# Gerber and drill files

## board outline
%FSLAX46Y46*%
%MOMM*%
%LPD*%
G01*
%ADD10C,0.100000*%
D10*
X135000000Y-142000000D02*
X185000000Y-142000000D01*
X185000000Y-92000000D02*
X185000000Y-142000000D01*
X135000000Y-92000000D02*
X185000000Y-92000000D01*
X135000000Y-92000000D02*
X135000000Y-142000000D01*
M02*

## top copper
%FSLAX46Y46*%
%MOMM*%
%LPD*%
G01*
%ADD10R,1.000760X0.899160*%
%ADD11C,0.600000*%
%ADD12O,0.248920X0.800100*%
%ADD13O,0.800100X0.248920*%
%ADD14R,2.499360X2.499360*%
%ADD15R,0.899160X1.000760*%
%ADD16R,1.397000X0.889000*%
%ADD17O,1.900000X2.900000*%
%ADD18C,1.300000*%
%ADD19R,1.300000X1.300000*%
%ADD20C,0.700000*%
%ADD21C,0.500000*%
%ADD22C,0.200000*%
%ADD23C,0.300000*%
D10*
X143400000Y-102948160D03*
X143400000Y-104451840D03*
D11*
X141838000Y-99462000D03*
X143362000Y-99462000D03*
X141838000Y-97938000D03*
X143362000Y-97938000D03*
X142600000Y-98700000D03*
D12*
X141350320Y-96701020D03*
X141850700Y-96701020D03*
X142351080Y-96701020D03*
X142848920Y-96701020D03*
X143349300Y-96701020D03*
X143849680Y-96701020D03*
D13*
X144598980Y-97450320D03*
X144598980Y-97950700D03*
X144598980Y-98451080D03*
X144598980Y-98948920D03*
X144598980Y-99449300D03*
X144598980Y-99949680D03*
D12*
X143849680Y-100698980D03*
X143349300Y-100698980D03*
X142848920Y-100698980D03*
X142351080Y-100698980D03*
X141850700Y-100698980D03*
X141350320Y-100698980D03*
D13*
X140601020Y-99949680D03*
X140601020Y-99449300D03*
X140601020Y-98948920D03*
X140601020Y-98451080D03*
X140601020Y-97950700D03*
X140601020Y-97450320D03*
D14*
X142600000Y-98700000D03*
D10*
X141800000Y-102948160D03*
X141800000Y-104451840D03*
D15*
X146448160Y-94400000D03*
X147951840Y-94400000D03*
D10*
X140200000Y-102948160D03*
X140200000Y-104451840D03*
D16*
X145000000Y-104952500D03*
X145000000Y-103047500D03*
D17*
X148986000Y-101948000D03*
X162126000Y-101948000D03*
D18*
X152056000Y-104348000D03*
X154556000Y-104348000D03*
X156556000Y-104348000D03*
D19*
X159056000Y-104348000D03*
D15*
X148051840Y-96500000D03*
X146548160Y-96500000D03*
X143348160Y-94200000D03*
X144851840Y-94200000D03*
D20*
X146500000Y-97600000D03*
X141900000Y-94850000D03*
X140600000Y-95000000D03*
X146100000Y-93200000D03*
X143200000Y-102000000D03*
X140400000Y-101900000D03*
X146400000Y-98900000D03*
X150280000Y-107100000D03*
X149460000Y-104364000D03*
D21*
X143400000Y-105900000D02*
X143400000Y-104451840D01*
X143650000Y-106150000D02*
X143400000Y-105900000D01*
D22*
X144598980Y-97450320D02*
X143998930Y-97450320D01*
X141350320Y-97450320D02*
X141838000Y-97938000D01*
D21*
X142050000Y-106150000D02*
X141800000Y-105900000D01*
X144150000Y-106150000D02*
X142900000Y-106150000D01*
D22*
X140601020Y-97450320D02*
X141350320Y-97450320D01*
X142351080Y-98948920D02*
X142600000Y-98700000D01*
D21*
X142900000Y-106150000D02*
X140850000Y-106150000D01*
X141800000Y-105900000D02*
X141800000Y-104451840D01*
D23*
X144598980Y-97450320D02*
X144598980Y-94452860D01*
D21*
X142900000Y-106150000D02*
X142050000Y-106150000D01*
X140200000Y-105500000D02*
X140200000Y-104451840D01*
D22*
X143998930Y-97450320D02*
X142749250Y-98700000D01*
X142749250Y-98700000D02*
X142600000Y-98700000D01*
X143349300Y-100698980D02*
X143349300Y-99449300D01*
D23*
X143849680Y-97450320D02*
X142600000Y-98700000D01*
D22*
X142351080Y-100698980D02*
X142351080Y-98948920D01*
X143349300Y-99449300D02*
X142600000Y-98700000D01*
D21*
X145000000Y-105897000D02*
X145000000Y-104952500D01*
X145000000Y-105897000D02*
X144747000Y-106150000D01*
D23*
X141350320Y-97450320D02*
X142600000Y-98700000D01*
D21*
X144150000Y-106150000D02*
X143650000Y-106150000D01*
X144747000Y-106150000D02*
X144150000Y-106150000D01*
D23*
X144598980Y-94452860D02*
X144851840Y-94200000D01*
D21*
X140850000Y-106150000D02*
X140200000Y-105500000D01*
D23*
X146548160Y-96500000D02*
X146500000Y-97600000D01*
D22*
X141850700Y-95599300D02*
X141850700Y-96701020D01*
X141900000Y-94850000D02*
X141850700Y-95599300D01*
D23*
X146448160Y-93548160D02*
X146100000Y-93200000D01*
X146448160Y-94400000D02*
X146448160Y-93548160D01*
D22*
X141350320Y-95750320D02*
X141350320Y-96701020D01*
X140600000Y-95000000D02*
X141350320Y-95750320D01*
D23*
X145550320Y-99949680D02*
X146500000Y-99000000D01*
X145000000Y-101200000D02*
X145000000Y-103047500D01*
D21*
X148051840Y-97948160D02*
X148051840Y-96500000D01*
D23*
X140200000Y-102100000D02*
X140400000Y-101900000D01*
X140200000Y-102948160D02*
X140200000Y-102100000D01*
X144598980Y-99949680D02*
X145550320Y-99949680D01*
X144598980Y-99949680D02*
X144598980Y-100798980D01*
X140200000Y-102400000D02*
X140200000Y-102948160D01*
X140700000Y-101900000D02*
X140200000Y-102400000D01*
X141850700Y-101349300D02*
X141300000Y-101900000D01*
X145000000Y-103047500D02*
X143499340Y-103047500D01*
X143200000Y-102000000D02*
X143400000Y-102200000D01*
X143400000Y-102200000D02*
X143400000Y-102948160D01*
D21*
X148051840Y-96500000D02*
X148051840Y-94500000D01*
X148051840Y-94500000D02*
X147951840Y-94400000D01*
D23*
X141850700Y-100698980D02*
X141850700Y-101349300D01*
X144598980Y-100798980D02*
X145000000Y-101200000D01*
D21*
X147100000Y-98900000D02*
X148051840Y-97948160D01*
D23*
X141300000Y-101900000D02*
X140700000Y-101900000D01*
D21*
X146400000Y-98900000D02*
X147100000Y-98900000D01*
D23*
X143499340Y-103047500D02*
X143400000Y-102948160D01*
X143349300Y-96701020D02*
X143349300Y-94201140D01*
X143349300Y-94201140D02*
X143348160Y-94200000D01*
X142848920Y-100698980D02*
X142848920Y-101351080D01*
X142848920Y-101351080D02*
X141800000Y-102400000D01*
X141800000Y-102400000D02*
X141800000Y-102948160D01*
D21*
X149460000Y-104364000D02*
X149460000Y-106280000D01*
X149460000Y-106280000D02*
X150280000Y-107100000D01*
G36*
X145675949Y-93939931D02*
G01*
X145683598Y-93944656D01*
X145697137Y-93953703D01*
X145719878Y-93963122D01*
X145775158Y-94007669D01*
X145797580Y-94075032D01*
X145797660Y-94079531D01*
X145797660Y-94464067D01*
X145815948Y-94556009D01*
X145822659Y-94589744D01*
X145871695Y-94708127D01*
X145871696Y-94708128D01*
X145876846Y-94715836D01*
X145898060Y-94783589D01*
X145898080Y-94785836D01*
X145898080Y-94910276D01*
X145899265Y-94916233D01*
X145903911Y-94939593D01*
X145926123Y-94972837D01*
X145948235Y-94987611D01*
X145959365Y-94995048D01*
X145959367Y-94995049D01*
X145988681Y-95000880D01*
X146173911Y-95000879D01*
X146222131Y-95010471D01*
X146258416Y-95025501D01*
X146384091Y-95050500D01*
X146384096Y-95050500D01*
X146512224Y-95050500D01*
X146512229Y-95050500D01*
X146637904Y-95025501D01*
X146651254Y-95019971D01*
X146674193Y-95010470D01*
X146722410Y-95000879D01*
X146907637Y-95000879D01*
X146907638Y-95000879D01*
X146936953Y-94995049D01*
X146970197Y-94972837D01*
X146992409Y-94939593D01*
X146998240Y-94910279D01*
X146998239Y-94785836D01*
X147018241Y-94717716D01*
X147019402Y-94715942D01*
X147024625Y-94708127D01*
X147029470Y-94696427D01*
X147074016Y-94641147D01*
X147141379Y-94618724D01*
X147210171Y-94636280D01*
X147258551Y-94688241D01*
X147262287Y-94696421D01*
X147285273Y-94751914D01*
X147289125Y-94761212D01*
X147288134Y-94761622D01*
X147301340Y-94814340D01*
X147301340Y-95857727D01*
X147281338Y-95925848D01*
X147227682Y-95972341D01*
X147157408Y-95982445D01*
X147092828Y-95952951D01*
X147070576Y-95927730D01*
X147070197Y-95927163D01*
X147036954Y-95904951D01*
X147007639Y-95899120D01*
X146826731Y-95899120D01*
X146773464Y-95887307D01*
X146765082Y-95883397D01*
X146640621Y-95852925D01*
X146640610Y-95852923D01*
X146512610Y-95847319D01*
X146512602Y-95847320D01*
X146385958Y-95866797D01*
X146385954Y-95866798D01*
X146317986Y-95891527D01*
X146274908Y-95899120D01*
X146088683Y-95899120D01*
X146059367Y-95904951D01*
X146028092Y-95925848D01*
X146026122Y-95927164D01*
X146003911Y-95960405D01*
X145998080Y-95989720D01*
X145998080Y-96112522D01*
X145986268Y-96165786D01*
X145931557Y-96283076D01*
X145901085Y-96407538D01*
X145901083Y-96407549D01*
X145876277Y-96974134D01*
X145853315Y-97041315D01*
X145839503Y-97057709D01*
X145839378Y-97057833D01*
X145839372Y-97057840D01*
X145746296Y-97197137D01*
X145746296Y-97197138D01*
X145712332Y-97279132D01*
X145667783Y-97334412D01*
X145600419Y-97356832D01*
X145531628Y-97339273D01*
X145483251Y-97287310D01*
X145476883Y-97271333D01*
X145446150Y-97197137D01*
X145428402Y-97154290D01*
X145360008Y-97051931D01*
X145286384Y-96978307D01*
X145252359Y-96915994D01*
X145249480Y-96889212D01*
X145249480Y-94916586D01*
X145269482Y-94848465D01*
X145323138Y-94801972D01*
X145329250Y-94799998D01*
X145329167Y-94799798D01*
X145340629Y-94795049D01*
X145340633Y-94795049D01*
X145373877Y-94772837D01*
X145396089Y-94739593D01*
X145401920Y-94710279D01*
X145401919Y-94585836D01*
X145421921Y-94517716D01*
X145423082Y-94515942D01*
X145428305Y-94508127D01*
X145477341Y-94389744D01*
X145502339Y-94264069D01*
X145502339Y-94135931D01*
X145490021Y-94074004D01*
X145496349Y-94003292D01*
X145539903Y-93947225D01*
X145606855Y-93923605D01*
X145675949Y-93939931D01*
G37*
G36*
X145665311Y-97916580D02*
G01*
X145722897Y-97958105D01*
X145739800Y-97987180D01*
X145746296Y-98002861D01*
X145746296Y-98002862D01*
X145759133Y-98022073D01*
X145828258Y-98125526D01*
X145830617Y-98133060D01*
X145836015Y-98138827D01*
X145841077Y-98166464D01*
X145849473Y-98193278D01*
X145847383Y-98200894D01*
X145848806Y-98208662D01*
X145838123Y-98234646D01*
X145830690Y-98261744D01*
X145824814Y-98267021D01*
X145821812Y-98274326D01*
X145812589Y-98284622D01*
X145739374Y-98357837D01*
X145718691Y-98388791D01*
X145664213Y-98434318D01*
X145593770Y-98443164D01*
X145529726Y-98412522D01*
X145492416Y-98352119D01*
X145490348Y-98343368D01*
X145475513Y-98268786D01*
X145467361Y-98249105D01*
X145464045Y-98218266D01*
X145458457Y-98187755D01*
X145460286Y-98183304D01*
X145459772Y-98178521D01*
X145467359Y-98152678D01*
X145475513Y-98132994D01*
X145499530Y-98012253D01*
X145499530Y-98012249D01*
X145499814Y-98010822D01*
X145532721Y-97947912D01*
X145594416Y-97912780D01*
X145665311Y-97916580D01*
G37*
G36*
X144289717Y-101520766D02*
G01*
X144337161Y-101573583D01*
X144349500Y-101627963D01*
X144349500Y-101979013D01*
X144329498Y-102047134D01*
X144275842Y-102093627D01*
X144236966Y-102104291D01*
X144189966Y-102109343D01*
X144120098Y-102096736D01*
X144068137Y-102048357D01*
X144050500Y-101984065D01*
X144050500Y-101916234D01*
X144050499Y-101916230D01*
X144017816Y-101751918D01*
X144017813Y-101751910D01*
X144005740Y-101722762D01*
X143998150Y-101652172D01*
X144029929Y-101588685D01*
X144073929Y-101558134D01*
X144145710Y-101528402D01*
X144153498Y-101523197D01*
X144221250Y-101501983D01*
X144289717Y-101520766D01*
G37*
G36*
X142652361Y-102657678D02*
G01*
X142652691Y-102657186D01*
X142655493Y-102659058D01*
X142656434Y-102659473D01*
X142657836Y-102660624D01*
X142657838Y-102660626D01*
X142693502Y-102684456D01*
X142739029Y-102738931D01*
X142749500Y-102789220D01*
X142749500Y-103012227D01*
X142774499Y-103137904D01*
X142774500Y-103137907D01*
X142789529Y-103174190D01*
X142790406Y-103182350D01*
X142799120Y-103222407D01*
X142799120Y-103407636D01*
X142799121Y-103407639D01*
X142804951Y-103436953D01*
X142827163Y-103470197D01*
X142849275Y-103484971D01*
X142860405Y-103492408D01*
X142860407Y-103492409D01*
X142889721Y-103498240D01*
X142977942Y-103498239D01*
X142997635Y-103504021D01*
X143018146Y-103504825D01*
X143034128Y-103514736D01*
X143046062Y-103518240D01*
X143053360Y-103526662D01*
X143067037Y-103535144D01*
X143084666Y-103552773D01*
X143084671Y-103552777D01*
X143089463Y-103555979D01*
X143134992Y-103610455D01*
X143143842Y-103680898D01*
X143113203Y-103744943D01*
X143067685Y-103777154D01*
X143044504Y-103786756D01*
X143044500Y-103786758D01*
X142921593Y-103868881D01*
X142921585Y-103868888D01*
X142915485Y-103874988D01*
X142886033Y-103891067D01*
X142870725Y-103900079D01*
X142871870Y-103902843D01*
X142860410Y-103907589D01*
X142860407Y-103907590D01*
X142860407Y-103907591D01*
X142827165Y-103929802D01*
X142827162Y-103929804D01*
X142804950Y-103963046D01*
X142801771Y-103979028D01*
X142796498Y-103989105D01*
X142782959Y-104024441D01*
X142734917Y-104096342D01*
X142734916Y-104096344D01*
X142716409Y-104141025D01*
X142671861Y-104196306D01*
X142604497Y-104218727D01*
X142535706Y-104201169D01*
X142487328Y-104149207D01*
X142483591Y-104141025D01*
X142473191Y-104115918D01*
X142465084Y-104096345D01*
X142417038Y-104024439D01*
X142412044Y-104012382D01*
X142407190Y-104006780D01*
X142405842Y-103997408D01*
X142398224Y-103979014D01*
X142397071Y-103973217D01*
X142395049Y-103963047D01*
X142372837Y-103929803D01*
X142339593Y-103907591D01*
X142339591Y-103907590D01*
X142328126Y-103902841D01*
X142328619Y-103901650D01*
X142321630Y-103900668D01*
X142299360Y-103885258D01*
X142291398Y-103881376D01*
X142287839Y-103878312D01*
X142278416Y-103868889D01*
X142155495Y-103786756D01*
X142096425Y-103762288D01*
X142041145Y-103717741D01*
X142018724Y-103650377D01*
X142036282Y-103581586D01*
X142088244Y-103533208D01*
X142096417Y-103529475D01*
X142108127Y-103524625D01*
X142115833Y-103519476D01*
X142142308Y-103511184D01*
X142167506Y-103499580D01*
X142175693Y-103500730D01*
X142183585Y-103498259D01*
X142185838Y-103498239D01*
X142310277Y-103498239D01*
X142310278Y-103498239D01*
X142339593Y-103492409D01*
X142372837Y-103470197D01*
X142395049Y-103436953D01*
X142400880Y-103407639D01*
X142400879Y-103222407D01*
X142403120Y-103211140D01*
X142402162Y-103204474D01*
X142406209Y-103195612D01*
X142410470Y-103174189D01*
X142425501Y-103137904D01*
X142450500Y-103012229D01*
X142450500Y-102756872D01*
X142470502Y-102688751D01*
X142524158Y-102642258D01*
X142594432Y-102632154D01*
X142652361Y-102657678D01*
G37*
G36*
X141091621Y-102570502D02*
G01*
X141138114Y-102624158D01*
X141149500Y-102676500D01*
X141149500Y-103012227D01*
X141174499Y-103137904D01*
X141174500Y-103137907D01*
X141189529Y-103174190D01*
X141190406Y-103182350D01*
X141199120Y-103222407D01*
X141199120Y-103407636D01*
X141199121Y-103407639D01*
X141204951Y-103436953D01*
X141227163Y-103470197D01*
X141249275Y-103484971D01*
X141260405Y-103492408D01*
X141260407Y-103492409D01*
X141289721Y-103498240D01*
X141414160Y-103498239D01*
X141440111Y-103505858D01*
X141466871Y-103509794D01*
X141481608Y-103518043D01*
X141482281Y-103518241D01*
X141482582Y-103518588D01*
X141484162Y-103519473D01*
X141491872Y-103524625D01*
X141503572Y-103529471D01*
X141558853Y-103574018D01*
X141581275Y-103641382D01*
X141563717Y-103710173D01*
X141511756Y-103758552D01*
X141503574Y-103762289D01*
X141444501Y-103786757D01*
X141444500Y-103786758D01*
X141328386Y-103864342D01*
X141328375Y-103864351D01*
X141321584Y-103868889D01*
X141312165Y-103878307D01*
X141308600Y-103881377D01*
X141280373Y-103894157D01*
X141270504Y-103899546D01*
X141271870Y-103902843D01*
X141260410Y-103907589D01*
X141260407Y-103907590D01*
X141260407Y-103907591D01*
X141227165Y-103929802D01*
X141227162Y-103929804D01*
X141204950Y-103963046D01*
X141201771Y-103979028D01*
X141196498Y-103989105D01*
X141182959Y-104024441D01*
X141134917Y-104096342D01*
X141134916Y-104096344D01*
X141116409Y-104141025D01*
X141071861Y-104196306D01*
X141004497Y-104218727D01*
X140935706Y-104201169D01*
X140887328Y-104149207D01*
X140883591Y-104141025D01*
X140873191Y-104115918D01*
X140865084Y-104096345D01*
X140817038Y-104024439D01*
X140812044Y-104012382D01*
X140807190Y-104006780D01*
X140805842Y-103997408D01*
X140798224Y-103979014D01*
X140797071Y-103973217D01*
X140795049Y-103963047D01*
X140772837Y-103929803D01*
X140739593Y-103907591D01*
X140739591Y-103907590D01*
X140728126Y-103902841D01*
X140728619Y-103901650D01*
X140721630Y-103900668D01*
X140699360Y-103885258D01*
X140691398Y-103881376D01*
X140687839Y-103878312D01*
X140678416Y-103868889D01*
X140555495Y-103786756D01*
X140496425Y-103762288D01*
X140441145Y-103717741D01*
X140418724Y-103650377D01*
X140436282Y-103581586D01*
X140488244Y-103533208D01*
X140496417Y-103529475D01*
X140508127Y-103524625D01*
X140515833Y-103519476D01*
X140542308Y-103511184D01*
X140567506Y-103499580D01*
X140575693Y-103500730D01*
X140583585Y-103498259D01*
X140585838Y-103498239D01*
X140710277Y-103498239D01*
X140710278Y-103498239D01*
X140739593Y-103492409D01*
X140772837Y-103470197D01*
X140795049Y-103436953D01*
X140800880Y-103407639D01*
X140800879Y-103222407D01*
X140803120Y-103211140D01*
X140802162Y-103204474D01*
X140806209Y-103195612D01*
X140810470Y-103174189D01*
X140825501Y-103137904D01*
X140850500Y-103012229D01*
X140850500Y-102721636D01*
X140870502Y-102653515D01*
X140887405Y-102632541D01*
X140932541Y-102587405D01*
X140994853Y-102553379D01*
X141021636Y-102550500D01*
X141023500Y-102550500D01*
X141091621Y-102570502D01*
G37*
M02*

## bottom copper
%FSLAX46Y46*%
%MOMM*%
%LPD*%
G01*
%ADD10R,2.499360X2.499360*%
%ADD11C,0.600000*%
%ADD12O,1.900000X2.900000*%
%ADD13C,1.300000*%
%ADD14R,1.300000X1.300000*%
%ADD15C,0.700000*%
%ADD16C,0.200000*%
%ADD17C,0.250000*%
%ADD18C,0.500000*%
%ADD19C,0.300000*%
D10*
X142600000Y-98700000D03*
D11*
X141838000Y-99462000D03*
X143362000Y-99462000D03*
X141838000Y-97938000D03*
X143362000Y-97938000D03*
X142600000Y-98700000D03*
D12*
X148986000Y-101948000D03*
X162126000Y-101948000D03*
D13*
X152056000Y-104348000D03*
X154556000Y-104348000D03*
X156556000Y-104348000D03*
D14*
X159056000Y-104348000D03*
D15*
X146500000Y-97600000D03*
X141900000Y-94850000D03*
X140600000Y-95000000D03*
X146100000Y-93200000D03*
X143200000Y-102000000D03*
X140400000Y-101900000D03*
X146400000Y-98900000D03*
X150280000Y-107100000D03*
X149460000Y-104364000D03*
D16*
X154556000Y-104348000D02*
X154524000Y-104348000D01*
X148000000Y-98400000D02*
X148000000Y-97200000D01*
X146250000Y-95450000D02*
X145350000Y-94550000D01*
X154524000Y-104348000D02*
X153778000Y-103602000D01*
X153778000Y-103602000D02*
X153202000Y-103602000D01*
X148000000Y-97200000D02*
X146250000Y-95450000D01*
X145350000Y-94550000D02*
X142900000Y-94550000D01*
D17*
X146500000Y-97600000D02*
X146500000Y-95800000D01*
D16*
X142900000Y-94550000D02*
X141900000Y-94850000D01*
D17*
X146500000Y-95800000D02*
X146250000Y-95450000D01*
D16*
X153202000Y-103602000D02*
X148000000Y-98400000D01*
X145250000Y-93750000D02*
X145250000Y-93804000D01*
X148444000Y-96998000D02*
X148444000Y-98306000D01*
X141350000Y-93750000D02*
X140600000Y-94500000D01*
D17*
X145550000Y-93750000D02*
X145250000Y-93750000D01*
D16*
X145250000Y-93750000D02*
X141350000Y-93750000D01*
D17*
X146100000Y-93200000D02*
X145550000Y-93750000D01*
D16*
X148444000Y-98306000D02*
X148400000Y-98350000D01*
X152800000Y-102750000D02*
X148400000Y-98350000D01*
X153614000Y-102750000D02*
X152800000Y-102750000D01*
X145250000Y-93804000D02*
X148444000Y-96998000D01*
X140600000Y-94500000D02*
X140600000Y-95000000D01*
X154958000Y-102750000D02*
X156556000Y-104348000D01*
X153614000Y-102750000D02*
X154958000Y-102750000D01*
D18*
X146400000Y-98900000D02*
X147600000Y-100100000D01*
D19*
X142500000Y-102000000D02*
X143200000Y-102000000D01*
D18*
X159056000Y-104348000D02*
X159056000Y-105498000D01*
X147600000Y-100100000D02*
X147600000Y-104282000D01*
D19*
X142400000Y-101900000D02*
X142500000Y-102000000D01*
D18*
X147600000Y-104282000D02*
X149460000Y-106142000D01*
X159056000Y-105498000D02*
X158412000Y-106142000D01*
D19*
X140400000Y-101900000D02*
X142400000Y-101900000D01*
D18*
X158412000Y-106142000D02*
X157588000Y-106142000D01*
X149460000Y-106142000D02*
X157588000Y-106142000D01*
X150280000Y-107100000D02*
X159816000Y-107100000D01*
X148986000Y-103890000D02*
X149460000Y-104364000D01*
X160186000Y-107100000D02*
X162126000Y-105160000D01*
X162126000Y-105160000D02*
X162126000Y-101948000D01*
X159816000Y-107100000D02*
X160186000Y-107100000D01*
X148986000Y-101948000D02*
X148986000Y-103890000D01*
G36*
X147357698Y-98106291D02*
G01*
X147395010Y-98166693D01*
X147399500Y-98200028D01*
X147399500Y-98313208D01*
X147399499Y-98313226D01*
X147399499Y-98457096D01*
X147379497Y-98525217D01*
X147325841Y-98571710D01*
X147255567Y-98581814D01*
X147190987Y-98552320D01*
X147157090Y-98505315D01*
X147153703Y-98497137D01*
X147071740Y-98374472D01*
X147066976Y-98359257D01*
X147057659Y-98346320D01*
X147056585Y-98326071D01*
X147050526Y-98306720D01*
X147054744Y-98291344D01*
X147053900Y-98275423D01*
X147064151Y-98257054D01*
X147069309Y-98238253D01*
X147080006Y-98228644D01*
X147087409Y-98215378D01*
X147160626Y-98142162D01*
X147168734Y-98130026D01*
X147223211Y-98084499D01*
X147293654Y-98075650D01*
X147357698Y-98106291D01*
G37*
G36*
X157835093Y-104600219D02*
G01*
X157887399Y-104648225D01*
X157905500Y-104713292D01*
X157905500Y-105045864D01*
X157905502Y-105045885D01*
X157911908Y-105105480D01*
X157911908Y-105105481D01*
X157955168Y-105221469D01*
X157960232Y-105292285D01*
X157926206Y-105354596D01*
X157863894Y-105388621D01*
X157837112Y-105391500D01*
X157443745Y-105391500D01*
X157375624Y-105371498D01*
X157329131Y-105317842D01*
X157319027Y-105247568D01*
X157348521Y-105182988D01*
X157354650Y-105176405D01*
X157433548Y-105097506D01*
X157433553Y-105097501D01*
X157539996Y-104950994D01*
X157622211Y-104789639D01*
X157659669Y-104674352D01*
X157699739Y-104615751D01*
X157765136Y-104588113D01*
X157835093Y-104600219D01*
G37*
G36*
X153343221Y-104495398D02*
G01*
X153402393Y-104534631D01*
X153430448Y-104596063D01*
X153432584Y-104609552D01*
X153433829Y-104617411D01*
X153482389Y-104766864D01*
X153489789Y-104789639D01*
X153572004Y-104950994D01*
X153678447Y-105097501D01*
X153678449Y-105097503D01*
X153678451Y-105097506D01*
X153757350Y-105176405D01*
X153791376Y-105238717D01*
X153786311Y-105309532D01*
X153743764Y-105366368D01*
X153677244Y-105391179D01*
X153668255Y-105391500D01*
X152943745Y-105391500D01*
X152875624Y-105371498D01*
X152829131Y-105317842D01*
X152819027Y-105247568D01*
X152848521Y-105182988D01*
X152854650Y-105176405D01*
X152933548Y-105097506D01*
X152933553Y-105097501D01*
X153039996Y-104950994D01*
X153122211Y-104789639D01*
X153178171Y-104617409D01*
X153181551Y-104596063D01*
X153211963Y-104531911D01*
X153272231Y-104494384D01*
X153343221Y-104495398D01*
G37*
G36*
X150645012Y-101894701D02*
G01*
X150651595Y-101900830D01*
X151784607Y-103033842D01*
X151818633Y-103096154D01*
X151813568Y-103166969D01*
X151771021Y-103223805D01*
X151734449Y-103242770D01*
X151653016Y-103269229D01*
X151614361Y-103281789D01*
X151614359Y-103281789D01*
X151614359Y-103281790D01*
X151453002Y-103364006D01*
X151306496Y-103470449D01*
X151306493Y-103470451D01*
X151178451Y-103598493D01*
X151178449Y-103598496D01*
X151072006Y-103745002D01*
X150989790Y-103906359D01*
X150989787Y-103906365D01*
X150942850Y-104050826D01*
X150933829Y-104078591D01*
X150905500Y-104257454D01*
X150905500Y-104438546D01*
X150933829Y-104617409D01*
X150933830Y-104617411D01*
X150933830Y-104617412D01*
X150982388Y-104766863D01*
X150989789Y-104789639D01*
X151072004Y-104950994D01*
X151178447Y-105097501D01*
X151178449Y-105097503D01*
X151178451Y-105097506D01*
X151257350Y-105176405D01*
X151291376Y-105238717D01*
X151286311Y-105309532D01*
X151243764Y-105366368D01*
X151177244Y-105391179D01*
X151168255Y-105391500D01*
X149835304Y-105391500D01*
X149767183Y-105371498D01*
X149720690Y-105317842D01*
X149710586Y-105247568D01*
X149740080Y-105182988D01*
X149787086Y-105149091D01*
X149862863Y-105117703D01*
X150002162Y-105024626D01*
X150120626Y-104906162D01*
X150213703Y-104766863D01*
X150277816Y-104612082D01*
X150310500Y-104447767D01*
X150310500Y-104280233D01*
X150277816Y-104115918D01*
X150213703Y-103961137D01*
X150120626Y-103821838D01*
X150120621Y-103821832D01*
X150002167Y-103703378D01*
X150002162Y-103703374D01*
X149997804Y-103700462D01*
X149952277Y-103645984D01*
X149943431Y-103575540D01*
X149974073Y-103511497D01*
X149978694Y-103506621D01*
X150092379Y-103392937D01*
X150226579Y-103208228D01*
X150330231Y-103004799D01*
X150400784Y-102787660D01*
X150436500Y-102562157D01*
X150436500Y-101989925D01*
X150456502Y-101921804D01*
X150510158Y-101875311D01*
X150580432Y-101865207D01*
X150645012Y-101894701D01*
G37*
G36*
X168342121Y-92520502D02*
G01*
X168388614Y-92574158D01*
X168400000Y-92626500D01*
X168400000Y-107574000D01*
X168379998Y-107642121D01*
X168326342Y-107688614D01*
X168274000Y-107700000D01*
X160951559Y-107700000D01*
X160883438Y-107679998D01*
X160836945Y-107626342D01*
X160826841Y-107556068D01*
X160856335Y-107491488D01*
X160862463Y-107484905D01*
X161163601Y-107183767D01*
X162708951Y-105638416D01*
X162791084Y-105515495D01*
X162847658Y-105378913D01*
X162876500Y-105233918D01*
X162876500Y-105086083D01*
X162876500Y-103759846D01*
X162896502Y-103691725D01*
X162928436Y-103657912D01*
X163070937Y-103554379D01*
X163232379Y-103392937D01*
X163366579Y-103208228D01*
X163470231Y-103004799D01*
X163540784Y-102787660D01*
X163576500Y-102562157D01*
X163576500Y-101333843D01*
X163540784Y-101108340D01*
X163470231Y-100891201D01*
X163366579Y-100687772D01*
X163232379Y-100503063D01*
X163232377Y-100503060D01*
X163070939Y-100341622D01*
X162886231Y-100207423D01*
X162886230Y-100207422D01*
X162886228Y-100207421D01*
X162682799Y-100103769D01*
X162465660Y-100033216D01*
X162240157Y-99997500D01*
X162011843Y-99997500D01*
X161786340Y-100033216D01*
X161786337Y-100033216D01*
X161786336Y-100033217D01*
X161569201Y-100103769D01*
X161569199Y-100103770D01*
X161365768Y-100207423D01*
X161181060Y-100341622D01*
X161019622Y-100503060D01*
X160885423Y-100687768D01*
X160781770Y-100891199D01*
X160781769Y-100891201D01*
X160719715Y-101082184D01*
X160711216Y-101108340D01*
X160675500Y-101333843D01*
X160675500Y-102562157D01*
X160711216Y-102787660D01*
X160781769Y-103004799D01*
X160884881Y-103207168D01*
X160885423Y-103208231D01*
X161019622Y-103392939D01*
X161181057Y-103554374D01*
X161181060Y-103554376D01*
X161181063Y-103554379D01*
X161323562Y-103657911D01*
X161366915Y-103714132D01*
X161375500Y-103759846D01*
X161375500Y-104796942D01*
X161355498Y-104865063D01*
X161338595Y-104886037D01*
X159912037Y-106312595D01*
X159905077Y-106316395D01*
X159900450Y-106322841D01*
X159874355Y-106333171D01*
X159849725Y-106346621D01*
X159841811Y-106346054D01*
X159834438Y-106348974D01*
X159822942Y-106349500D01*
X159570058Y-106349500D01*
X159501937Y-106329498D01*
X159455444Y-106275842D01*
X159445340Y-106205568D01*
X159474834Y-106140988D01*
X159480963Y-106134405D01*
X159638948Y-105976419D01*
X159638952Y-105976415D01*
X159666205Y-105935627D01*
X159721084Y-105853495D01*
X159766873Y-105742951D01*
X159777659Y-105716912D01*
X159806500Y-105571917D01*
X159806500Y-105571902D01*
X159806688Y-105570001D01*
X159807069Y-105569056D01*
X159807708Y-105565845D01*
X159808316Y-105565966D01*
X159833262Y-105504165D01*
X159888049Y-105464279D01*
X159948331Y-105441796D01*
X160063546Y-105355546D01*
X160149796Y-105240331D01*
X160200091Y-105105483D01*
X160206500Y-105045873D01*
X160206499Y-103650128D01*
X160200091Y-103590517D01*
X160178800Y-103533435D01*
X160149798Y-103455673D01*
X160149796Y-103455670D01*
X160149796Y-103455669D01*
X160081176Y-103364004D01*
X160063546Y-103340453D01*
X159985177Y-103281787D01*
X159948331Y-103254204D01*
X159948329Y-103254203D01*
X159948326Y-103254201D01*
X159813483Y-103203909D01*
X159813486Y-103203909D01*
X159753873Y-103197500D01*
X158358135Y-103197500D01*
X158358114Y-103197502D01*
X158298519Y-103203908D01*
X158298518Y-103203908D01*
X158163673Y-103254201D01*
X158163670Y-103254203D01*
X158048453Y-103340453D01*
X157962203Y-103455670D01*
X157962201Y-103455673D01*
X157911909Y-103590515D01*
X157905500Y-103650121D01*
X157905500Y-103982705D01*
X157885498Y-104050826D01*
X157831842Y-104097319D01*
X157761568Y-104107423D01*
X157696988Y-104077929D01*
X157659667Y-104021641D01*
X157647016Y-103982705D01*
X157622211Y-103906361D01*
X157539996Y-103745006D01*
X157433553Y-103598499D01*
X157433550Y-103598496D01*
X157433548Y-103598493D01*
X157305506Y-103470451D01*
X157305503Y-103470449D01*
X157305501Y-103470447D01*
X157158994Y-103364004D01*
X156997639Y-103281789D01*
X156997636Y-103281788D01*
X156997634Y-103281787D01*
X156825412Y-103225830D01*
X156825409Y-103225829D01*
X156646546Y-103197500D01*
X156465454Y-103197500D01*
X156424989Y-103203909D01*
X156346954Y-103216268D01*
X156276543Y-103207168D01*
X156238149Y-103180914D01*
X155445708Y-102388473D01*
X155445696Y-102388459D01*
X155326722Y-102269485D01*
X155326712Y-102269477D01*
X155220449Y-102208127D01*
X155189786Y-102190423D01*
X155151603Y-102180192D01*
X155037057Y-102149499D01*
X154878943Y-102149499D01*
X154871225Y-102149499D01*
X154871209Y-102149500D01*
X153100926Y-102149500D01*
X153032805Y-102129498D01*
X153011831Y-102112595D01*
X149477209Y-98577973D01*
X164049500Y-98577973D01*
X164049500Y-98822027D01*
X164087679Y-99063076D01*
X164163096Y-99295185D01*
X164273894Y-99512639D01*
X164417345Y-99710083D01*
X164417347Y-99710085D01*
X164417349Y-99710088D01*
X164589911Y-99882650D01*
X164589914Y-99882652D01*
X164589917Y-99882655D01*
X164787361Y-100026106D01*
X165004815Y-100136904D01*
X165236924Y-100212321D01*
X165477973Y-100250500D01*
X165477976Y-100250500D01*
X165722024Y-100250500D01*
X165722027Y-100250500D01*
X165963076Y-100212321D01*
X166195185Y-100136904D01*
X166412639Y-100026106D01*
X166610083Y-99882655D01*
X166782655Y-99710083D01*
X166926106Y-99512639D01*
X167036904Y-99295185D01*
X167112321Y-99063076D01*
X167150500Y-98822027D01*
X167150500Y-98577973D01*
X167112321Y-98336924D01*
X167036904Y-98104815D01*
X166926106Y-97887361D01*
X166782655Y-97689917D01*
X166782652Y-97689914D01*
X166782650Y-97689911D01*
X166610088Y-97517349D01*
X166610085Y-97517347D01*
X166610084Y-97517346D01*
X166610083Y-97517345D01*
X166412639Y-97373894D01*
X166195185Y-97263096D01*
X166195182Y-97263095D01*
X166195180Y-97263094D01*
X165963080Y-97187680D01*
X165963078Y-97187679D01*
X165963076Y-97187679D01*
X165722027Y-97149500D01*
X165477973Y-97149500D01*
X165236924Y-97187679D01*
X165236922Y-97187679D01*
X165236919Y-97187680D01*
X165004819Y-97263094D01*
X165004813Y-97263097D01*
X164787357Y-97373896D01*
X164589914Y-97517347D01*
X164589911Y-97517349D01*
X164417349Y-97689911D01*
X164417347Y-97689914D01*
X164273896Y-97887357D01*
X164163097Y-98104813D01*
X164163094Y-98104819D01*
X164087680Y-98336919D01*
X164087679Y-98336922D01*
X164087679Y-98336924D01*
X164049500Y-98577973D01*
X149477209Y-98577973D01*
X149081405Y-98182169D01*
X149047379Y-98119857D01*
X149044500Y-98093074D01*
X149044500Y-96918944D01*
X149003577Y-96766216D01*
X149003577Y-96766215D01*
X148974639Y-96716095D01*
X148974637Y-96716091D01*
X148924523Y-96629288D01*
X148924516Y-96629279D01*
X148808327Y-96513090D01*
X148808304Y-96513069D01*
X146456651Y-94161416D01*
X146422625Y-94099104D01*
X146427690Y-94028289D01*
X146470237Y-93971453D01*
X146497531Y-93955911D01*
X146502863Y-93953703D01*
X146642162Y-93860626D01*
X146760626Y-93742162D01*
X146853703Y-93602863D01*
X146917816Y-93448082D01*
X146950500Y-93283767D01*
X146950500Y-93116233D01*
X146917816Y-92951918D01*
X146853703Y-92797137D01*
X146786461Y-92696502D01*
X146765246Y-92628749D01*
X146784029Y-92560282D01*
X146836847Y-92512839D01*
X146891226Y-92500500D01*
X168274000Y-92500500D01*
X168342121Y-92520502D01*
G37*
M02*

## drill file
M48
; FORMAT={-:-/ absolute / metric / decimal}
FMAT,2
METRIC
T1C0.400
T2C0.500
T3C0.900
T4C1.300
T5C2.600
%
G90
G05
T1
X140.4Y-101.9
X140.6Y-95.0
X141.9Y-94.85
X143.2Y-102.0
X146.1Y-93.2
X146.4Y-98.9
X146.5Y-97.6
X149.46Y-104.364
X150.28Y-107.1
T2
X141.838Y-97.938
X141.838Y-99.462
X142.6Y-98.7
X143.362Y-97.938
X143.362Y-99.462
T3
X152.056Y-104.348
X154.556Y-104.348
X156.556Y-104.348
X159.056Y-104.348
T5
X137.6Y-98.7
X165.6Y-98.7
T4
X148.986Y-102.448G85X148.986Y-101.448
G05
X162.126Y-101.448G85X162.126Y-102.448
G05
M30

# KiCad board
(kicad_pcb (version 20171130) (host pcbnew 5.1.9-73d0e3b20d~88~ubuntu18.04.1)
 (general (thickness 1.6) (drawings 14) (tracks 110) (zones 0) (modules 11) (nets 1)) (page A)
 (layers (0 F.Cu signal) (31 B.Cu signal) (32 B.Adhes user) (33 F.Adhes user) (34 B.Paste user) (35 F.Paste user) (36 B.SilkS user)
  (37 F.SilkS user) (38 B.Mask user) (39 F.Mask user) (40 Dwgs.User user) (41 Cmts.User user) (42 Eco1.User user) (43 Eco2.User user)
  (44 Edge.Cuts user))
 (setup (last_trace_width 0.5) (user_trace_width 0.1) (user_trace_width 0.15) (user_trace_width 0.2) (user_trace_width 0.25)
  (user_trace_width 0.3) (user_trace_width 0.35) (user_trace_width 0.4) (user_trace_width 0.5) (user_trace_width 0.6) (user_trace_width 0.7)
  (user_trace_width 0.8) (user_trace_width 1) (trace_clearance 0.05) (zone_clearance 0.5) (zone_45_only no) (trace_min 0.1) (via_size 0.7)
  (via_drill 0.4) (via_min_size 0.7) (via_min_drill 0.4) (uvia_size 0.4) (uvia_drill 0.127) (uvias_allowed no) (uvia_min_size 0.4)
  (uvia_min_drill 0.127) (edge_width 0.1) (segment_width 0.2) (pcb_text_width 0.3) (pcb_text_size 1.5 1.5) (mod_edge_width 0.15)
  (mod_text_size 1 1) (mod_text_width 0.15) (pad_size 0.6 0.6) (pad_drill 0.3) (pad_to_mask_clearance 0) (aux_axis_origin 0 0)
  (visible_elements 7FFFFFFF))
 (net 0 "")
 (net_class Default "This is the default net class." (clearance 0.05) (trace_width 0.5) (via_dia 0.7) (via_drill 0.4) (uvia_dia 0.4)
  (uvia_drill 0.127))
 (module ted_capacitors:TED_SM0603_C (layer F.Cu) (at 143.4 103.7 270)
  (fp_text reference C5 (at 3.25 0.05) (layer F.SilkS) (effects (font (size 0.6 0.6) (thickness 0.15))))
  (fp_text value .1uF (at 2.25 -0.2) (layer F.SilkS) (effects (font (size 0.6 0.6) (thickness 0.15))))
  (pad 1 smd rect (at -0.75184 0 270) (size 0.89916 1.00076) (layers F.Cu F.Paste F.Mask) (clearance 0.1))
  (pad 2 smd rect (at 0.75184 0 270) (size 0.89916 1.00076) (layers F.Cu F.Paste F.Mask) (clearance 0.1)))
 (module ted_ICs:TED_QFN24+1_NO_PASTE (layer F.Cu) (at 142.6 98.7)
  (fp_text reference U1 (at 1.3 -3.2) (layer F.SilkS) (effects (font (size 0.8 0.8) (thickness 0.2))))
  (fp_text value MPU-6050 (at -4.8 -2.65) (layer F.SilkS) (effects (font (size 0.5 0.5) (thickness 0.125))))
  (pad 25 smd rect (at 0 0 270) (size 2.49936 2.49936) (layers B.Cu B.Mask) (zone_connect 2))
  (pad 25 thru_hole circle (at -0.762 0.762 270) (size 0.6 0.6) (drill 0.5) (layers *.Cu) (zone_connect 2))
  (pad 25 thru_hole circle (at 0.762 0.762 270) (size 0.6 0.6) (drill 0.5) (layers *.Cu) (zone_connect 2))
  (pad 25 thru_hole circle (at -0.762 -0.762 270) (size 0.6 0.6) (drill 0.5) (layers *.Cu) (zone_connect 2))
  (pad 25 thru_hole circle (at 0.762 -0.762 270) (size 0.6 0.6) (drill 0.5) (layers *.Cu) (zone_connect 2))
  (pad 25 thru_hole circle (at 0 0 270) (size 0.6 0.6) (drill 0.5) (layers *.Cu) (zone_connect 2))
  (pad 24 smd oval (at -1.24968 -1.99898 270) (size 0.8001 0.24892) (layers F.Cu F.Paste F.Mask))
  (pad 23 smd oval (at -0.7493 -1.99898 270) (size 0.8001 0.24892) (layers F.Cu F.Paste F.Mask))
  (pad 22 smd oval (at -0.24892 -1.99898 270) (size 0.8001 0.24892) (layers F.Cu F.Paste F.Mask))
  (pad 21 smd oval (at 0.24892 -1.99898 270) (size 0.8001 0.24892) (layers F.Cu F.Paste F.Mask))
  (pad 20 smd oval (at 0.7493 -1.99898 270) (size 0.8001 0.24892) (layers F.Cu F.Paste F.Mask))
  (pad 19 smd oval (at 1.24968 -1.99898 270) (size 0.8001 0.24892) (layers F.Cu F.Paste F.Mask))
  (pad 18 smd oval (at 1.99898 -1.24968 180) (size 0.8001 0.24892) (layers F.Cu F.Paste F.Mask))
  (pad 17 smd oval (at 1.99898 -0.7493 180) (size 0.8001 0.24892) (layers F.Cu F.Paste F.Mask))
  (pad 16 smd oval (at 1.99898 -0.24892 180) (size 0.8001 0.24892) (layers F.Cu F.Paste F.Mask))
  (pad 15 smd oval (at 1.99898 0.24892 180) (size 0.8001 0.24892) (layers F.Cu F.Paste F.Mask))
  (pad 14 smd oval (at 1.99898 0.7493 180) (size 0.8001 0.24892) (layers F.Cu F.Paste F.Mask))
  (pad 13 smd oval (at 1.99898 1.24968 180) (size 0.8001 0.24892) (layers F.Cu F.Paste F.Mask))
  (pad 12 smd oval (at 1.24968 1.99898 90) (size 0.8001 0.24892) (layers F.Cu F.Paste F.Mask))
  (pad 11 smd oval (at 0.7493 1.99898 90) (size 0.8001 0.24892) (layers F.Cu F.Paste F.Mask))
  (pad 10 smd oval (at 0.24892 1.99898 90) (size 0.8001 0.24892) (layers F.Cu F.Paste F.Mask))
  (pad 9 smd oval (at -0.24892 1.99898 90) (size 0.8001 0.24892) (layers F.Cu F.Paste F.Mask))
  (pad 8 smd oval (at -0.7493 1.99898 90) (size 0.8001 0.24892) (layers F.Cu F.Paste F.Mask))
  (pad 7 smd oval (at -1.24968 1.99898 90) (size 0.8001 0.24892) (layers F.Cu F.Paste F.Mask))
  (pad 6 smd oval (at -1.99898 1.24968) (size 0.8001 0.24892) (layers F.Cu F.Paste F.Mask))
  (pad 5 smd oval (at -1.99898 0.7493) (size 0.8001 0.24892) (layers F.Cu F.Paste F.Mask))
  (pad 4 smd oval (at -1.99898 0.24892) (size 0.8001 0.24892) (layers F.Cu F.Paste F.Mask))
  (pad 3 smd oval (at -1.99898 -0.24892) (size 0.8001 0.24892) (layers F.Cu F.Paste F.Mask))
  (pad 2 smd oval (at -1.99898 -0.7493) (size 0.8001 0.24892) (layers F.Cu F.Paste F.Mask))
  (pad 1 smd oval (at -1.99898 -1.24968) (size 0.8001 0.24892) (layers F.Cu F.Paste F.Mask))
  (pad 25 smd rect (at 0 0 270) (size 2.49936 2.49936) (layers F.Cu F.Mask) (zone_connect 2)))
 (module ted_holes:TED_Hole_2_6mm (layer F.Cu) (at 165.6 98.7)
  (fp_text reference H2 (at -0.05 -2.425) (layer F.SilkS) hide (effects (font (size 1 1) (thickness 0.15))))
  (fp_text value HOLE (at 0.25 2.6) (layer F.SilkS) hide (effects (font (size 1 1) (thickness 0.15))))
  (pad "" np_thru_hole circle (at 0 0) (size 2.6 2.6) (drill 2.6) (layers *.Cu *.Mask F.SilkS)))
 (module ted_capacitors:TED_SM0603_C (layer F.Cu) (at 141.8 103.7 270)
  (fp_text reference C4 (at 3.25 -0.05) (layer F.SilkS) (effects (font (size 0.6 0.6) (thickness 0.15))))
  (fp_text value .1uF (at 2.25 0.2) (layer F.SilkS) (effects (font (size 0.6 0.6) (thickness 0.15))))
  (pad 1 smd rect (at -0.75184 0 270) (size 0.89916 1.00076) (layers F.Cu F.Paste F.Mask) (clearance 0.1))
  (pad 2 smd rect (at 0.75184 0 270) (size 0.89916 1.00076) (layers F.Cu F.Paste F.Mask) (clearance 0.1)))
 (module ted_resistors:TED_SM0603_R (layer F.Cu) (at 147.2 94.4 180)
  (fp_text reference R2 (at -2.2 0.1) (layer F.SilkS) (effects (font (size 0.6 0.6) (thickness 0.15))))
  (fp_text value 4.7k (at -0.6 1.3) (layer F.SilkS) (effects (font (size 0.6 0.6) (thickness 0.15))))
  (pad 2 smd rect (at 0.75184 0 180) (size 0.89916 1.00076) (layers F.Cu F.Paste F.Mask) (clearance 0.1))
  (pad 1 smd rect (at -0.75184 0 180) (size 0.89916 1.00076) (layers F.Cu F.Paste F.Mask) (clearance 0.1)))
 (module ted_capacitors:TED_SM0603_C (layer F.Cu) (at 140.2 103.7 270)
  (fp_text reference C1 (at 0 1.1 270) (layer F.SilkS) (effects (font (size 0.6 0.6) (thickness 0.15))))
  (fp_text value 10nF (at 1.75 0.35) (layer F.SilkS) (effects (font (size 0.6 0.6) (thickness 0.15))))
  (pad 1 smd rect (at -0.75184 0 270) (size 0.89916 1.00076) (layers F.Cu F.Paste F.Mask) (clearance 0.1))
  (pad 2 smd rect (at 0.75184 0 270) (size 0.89916 1.00076) (layers F.Cu F.Paste F.Mask) (clearance 0.1)))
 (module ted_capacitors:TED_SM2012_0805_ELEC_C (layer F.Cu) (at 145 104 270)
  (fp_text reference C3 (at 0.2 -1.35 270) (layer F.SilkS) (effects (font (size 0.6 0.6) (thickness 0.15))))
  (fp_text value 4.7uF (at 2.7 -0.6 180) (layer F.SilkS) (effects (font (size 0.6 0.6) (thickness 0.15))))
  (pad 2 smd rect (at 0.9525 0 270) (size 0.889 1.397) (layers F.Cu F.Paste F.Mask))
  (pad 1 smd rect (at -0.9525 0 270) (size 0.889 1.397) (layers F.Cu F.Paste F.Mask)))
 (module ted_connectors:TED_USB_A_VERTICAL (layer F.Cu) (at 155.556 103.348 180)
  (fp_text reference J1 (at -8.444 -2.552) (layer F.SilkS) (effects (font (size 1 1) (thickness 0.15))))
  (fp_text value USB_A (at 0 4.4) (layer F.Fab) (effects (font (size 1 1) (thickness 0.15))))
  (pad 5 thru_hole oval (at 6.57 1.4 180) (size 1.9 2.9) (drill oval 1.3 2.3) (layers *.Cu *.Mask))
  (pad 5 thru_hole oval (at -6.57 1.4) (size 1.9 2.9) (drill oval 1.3 2.3) (layers *.Cu *.Mask))
  (pad 4 thru_hole circle (at 3.5 -1 180) (size 1.3 1.3) (drill 0.9) (layers *.Cu *.Mask))
  (pad 3 thru_hole circle (at 1 -1 180) (size 1.3 1.3) (drill 0.9) (layers *.Cu *.Mask))
  (pad 2 thru_hole circle (at -1 -1 180) (size 1.3 1.3) (drill 0.9) (layers *.Cu *.Mask))
  (pad 1 thru_hole rect (at -3.5 -1 180) (size 1.3 1.3) (drill 0.9) (layers *.Cu *.Mask)))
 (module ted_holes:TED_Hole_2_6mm (layer F.Cu) (at 137.6 98.7)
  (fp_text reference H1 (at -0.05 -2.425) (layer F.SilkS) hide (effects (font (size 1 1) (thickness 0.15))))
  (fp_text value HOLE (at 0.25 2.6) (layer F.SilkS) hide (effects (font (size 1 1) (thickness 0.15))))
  (pad "" np_thru_hole circle (at 0 0) (size 2.6 2.6) (drill 2.6) (layers *.Cu *.Mask F.SilkS)))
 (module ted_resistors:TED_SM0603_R (layer F.Cu) (at 147.3 96.5 180)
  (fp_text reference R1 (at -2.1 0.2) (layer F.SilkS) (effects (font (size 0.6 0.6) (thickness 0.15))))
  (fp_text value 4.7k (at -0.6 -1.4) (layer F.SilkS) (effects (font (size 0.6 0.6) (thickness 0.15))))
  (pad 1 smd rect (at -0.75184 0 180) (size 0.89916 1.00076) (layers F.Cu F.Paste F.Mask) (clearance 0.1))
  (pad 2 smd rect (at 0.75184 0 180) (size 0.89916 1.00076) (layers F.Cu F.Paste F.Mask) (clearance 0.1)))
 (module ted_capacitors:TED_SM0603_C (layer F.Cu) (at 144.1 94.2)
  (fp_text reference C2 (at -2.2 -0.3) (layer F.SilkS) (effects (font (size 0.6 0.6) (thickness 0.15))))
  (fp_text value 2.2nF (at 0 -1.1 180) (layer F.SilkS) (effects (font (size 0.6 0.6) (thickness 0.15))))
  (pad 1 smd rect (at -0.75184 0) (size 0.89916 1.00076) (layers F.Cu F.Paste F.Mask) (clearance 0.1))
  (pad 2 smd rect (at 0.75184 0) (size 0.89916 1.00076) (layers F.Cu F.Paste F.Mask) (clearance 0.1)))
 (gr_line (start 135 142) (end 185 142) (angle 90) (layer Edge.Cuts) (width 0.1))
 (gr_line (start 185 92) (end 185 142) (angle 90) (layer Edge.Cuts) (width 0.1))
 (gr_line (start 135 92) (end 185 92) (angle 90) (layer Edge.Cuts) (width 0.1))
 (gr_line (start 135 92) (end 135 142) (angle 90) (layer Edge.Cuts) (width 0.1))
 (segment (start 143.4 105.9) (end 143.4 104.45184) (width 0.5) (layer F.Cu) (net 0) (status 20))
 (segment (start 143.65 106.15) (end 143.4 105.9) (width 0.5) (layer F.Cu) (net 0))
 (segment (start 144.59898 97.45032) (end 143.99893 97.45032) (width 0.2) (layer F.Cu) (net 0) (status 10))
 (segment (start 141.35032 97.45032) (end 141.838 97.938) (width 0.2) (layer F.Cu) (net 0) (status 30))
 (segment (start 142.05 106.15) (end 141.8 105.9) (width 0.5) (layer F.Cu) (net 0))
 (segment (start 144.15 106.15) (end 142.9 106.15) (width 0.5) (layer F.Cu) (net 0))
 (segment (start 140.60102 97.45032) (end 141.35032 97.45032) (width 0.2) (layer F.Cu) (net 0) (status 30))
 (segment (start 142.35108 98.94892) (end 142.6 98.7) (width 0.2) (layer F.Cu) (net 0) (status 30))
 (segment (start 142.9 106.15) (end 140.85 106.15) (width 0.5) (layer F.Cu) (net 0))
 (segment (start 141.8 105.9) (end 141.8 104.45184) (width 0.5) (layer F.Cu) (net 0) (status 20))
 (segment (start 144.59898 97.45032) (end 144.59898 94.45286) (width 0.3) (layer F.Cu) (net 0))
 (segment (start 142.9 106.15) (end 142.05 106.15) (width 0.5) (layer F.Cu) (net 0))
 (segment (start 140.2 105.5) (end 140.2 104.45184) (width 0.5) (layer F.Cu) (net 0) (status 20))
 (segment (start 143.99893 97.45032) (end 142.74925 98.7) (width 0.2) (layer F.Cu) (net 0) (status 20))
 (segment (start 142.74925 98.7) (end 142.6 98.7) (width 0.2) (layer F.Cu) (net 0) (status 30))
 (segment (start 143.3493 100.69898) (end 143.3493 99.4493) (width 0.2) (layer F.Cu) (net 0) (status 30))
 (segment (start 143.84968 97.45032) (end 142.6 98.7) (width 0.3) (layer F.Cu) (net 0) (status 30))
 (segment (start 142.35108 100.69898) (end 142.35108 98.94892) (width 0.2) (layer F.Cu) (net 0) (status 30))
 (segment (start 143.3493 99.4493) (end 142.6 98.7) (width 0.2) (layer F.Cu) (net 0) (status 30))
 (segment (start 145 105.897) (end 145 104.9525) (width 0.5) (layer F.Cu) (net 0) (status 20))
 (segment (start 145 105.897) (end 144.747 106.15) (width 0.5) (layer F.Cu) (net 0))
 (segment (start 141.35032 97.45032) (end 142.6 98.7) (width 0.3) (layer F.Cu) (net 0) (status 30))
 (segment (start 144.15 106.15) (end 143.65 106.15) (width 0.5) (layer F.Cu) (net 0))
 (segment (start 144.747 106.15) (end 144.15 106.15) (width 0.5) (layer F.Cu) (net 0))
 (segment (start 144.59898 94.45286) (end 144.85184 94.2) (width 0.3) (layer F.Cu) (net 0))
 (segment (start 140.85 106.15) (end 140.2 105.5) (width 0.5) (layer F.Cu) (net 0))
 (via (at 146.5 97.6) (size 0.7) (drill 0.4) (layers F.Cu B.Cu) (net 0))
 (segment (start 154.556 104.348) (end 154.524 104.348) (width 0.2) (layer B.Cu) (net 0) (status 30))
 (segment (start 148 98.4) (end 148 97.2) (width 0.2) (layer B.Cu) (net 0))
 (segment (start 146.25 95.45) (end 145.35 94.55) (width 0.2) (layer B.Cu) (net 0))
 (segment (start 154.524 104.348) (end 153.778 103.602) (width 0.2) (layer B.Cu) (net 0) (status 10))
 (segment (start 146.54816 96.5) (end 146.5 97.6) (width 0.3) (layer F.Cu) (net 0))
 (segment (start 153.778 103.602) (end 153.202 103.602) (width 0.2) (layer B.Cu) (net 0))
 (segment (start 148 97.2) (end 146.25 95.45) (width 0.2) (layer B.Cu) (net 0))
 (via (at 141.9 94.85) (size 0.7) (drill 0.4) (layers F.Cu B.Cu) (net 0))
 (segment (start 145.35 94.55) (end 142.9 94.55) (width 0.2) (layer B.Cu) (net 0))
 (segment (start 146.5 97.6) (end 146.5 95.8) (width 0.25) (layer B.Cu) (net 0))
 (segment (start 142.9 94.55) (end 141.9 94.85) (width 0.2) (layer B.Cu) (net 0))
 (segment (start 141.8507 95.5993) (end 141.8507 96.70102) (width 0.2) (layer F.Cu) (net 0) (status 20))
 (segment (start 146.5 95.8) (end 146.25 95.45) (width 0.25) (layer B.Cu) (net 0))
 (segment (start 141.9 94.85) (end 141.8507 95.5993) (width 0.2) (layer F.Cu) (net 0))
 (segment (start 153.202 103.602) (end 148 98.4) (width 0.2) (layer B.Cu) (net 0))
 (segment (start 145.25 93.75) (end 145.25 93.804) (width 0.2) (layer B.Cu) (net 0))
 (segment (start 148.444 96.998) (end 148.444 98.306) (width 0.2) (layer B.Cu) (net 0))
 (segment (start 141.35 93.75) (end 140.6 94.5) (width 0.2) (layer B.Cu) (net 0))
 (segment (start 145.55 93.75) (end 145.25 93.75) (width 0.25) (layer B.Cu) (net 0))
 (segment (start 145.25 93.75) (end 141.35 93.75) (width 0.2) (layer B.Cu) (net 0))
 (via (at 140.6 95) (size 0.7) (drill 0.4) (layers F.Cu B.Cu) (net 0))
 (segment (start 146.44816 93.54816) (end 146.1 93.2) (width 0.3) (layer F.Cu) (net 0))
 (segment (start 146.1 93.2) (end 145.55 93.75) (width 0.25) (layer B.Cu) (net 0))
 (segment (start 148.444 98.306) (end 148.4 98.35) (width 0.2) (layer B.Cu) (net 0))
 (segment (start 152.8 102.75) (end 148.4 98.35) (width 0.2) (layer B.Cu) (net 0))
 (segment (start 146.44816 94.4) (end 146.44816 93.54816) (width 0.3) (layer F.Cu) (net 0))
 (segment (start 141.35032 95.75032) (end 141.35032 96.70102) (width 0.2) (layer F.Cu) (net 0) (status 20))
 (segment (start 140.6 95) (end 141.35032 95.75032) (width 0.2) (layer F.Cu) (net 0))
 (segment (start 153.614 102.75) (end 152.8 102.75) (width 0.2) (layer B.Cu) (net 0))
 (segment (start 145.25 93.804) (end 148.444 96.998) (width 0.2) (layer B.Cu) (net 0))
 (segment (start 140.6 94.5) (end 140.6 95) (width 0.2) (layer B.Cu) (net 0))
 (segment (start 154.958 102.75) (end 156.556 104.348) (width 0.2) (layer B.Cu) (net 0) (status 20))
 (via (at 146.1 93.2) (size 0.7) (drill 0.4) (layers F.Cu B.Cu) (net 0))
 (segment (start 153.614 102.75) (end 154.958 102.75) (width 0.2) (layer B.Cu) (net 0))
 (segment (start 145.55032 99.94968) (end 146.5 99) (width 0.3) (layer F.Cu) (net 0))
 (segment (start 145 101.2) (end 145 103.0475) (width 0.3) (layer F.Cu) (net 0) (status 20))
 (segment (start 148.05184 97.94816) (end 148.05184 96.5) (width 0.5) (layer F.Cu) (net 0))
 (segment (start 146.4 98.9) (end 147.6 100.1) (width 0.5) (layer B.Cu) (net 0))
 (segment (start 140.2 102.1) (end 140.4 101.9) (width 0.3) (layer F.Cu) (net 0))
 (segment (start 140.2 102.94816) (end 140.2 102.1) (width 0.3) (layer F.Cu) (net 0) (status 10))
 (segment (start 142.5 102) (end 143.2 102) (width 0.3) (layer B.Cu) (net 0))
 (via (at 143.2 102) (size 0.7) (drill 0.4) (layers F.Cu B.Cu) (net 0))
 (segment (start 159.056 104.348) (end 159.056 105.498) (width 0.5) (layer B.Cu) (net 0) (status 10))
 (segment (start 144.59898 99.94968) (end 145.55032 99.94968) (width 0.3) (layer F.Cu) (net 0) (status 10))
 (segment (start 144.59898 99.94968) (end 144.59898 100.79898) (width 0.3) (layer F.Cu) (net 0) (status 10))
 (segment (start 147.6 100.1) (end 147.6 104.282) (width 0.5) (layer B.Cu) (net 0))
 (segment (start 142.4 101.9) (end 142.5 102) (width 0.3) (layer B.Cu) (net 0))
 (segment (start 147.6 104.282) (end 149.46 106.142) (width 0.5) (layer B.Cu) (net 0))
 (segment (start 159.056 105.498) (end 158.412 106.142) (width 0.5) (layer B.Cu) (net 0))
 (segment (start 140.4 101.9) (end 142.4 101.9) (width 0.3) (layer B.Cu) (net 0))
 (segment (start 140.2 102.4) (end 140.2 102.94816) (width 0.3) (layer F.Cu) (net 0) (status 20))
 (segment (start 140.7 101.9) (end 140.2 102.4) (width 0.3) (layer F.Cu) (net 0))
 (segment (start 141.8507 101.3493) (end 141.3 101.9) (width 0.3) (layer F.Cu) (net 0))
 (segment (start 145 103.0475) (end 143.49934 103.0475) (width 0.3) (layer F.Cu) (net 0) (status 30))
 (segment (start 143.2 102) (end 143.4 102.2) (width 0.3) (layer F.Cu) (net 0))
 (segment (start 143.4 102.2) (end 143.4 102.94816) (width 0.3) (layer F.Cu) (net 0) (status 20))
 (segment (start 158.412 106.142) (end 157.588 106.142) (width 0.5) (layer B.Cu) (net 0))
 (segment (start 148.05184 96.5) (end 148.05184 94.5) (width 0.5) (layer F.Cu) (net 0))
 (via (at 140.4 101.9) (size 0.7) (drill 0.4) (layers F.Cu B.Cu) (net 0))
 (segment (start 148.05184 94.5) (end 147.95184 94.4) (width 0.5) (layer F.Cu) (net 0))
 (segment (start 141.8507 100.69898) (end 141.8507 101.3493) (width 0.3) (layer F.Cu) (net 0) (status 10))
 (segment (start 149.46 106.142) (end 157.588 106.142) (width 0.5) (layer B.Cu) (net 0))
 (segment (start 144.59898 100.79898) (end 145 101.2) (width 0.3) (layer F.Cu) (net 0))
 (segment (start 147.1 98.9) (end 148.05184 97.94816) (width 0.5) (layer F.Cu) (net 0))
 (via (at 146.4 98.9) (size 0.7) (drill 0.4) (layers F.Cu B.Cu) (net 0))
 (segment (start 141.3 101.9) (end 140.7 101.9) (width 0.3) (layer F.Cu) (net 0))
 (segment (start 146.4 98.9) (end 147.1 98.9) (width 0.5) (layer F.Cu) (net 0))
 (segment (start 143.49934 103.0475) (end 143.4 102.94816) (width 0.3) (layer F.Cu) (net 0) (status 30))
 (segment (start 143.3493 96.70102) (end 143.3493 94.20114) (width 0.3) (layer F.Cu) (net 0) (status 30))
 (segment (start 143.3493 94.20114) (end 143.34816 94.2) (width 0.3) (layer F.Cu) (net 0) (status 30))
 (segment (start 142.84892 100.69898) (end 142.84892 101.35108) (width 0.3) (layer F.Cu) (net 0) (status 10))
 (segment (start 142.84892 101.35108) (end 141.8 102.4) (width 0.3) (layer F.Cu) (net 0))
 (segment (start 141.8 102.4) (end 141.8 102.94816) (width 0.3) (layer F.Cu) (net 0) (status 20))
 (segment (start 150.28 107.1) (end 159.816 107.1) (width 0.5) (layer B.Cu) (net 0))
 (segment (start 148.986 103.89) (end 149.46 104.364) (width 0.5) (layer B.Cu) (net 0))
 (segment (start 149.46 104.364) (end 149.46 106.28) (width 0.5) (layer F.Cu) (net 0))
 (segment (start 160.186 107.1) (end 162.126 105.16) (width 0.5) (layer B.Cu) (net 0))
 (via (at 150.28 107.1) (size 0.7) (drill 0.4) (layers F.Cu B.Cu) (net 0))
 (segment (start 162.126 105.16) (end 162.126 101.948) (width 0.5) (layer B.Cu) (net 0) (status 20))
 (segment (start 159.816 107.1) (end 160.186 107.1) (width 0.5) (layer B.Cu) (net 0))
 (segment (start 149.46 106.28) (end 150.28 107.1) (width 0.5) (layer F.Cu) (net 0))
 (segment (start 148.986 101.948) (end 148.986 103.89) (width 0.5) (layer B.Cu) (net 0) (status 10))
 (via (at 149.46 104.364) (size 0.7) (drill 0.4) (layers F.Cu B.Cu) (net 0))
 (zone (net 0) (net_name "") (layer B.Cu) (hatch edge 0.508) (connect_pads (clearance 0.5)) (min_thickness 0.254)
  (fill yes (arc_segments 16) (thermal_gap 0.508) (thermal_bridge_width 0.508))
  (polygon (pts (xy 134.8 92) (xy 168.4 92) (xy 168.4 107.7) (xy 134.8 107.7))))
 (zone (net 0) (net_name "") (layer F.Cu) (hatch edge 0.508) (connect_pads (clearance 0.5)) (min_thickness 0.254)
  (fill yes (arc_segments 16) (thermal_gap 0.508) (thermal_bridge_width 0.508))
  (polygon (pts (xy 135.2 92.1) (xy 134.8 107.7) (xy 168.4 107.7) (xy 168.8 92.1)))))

